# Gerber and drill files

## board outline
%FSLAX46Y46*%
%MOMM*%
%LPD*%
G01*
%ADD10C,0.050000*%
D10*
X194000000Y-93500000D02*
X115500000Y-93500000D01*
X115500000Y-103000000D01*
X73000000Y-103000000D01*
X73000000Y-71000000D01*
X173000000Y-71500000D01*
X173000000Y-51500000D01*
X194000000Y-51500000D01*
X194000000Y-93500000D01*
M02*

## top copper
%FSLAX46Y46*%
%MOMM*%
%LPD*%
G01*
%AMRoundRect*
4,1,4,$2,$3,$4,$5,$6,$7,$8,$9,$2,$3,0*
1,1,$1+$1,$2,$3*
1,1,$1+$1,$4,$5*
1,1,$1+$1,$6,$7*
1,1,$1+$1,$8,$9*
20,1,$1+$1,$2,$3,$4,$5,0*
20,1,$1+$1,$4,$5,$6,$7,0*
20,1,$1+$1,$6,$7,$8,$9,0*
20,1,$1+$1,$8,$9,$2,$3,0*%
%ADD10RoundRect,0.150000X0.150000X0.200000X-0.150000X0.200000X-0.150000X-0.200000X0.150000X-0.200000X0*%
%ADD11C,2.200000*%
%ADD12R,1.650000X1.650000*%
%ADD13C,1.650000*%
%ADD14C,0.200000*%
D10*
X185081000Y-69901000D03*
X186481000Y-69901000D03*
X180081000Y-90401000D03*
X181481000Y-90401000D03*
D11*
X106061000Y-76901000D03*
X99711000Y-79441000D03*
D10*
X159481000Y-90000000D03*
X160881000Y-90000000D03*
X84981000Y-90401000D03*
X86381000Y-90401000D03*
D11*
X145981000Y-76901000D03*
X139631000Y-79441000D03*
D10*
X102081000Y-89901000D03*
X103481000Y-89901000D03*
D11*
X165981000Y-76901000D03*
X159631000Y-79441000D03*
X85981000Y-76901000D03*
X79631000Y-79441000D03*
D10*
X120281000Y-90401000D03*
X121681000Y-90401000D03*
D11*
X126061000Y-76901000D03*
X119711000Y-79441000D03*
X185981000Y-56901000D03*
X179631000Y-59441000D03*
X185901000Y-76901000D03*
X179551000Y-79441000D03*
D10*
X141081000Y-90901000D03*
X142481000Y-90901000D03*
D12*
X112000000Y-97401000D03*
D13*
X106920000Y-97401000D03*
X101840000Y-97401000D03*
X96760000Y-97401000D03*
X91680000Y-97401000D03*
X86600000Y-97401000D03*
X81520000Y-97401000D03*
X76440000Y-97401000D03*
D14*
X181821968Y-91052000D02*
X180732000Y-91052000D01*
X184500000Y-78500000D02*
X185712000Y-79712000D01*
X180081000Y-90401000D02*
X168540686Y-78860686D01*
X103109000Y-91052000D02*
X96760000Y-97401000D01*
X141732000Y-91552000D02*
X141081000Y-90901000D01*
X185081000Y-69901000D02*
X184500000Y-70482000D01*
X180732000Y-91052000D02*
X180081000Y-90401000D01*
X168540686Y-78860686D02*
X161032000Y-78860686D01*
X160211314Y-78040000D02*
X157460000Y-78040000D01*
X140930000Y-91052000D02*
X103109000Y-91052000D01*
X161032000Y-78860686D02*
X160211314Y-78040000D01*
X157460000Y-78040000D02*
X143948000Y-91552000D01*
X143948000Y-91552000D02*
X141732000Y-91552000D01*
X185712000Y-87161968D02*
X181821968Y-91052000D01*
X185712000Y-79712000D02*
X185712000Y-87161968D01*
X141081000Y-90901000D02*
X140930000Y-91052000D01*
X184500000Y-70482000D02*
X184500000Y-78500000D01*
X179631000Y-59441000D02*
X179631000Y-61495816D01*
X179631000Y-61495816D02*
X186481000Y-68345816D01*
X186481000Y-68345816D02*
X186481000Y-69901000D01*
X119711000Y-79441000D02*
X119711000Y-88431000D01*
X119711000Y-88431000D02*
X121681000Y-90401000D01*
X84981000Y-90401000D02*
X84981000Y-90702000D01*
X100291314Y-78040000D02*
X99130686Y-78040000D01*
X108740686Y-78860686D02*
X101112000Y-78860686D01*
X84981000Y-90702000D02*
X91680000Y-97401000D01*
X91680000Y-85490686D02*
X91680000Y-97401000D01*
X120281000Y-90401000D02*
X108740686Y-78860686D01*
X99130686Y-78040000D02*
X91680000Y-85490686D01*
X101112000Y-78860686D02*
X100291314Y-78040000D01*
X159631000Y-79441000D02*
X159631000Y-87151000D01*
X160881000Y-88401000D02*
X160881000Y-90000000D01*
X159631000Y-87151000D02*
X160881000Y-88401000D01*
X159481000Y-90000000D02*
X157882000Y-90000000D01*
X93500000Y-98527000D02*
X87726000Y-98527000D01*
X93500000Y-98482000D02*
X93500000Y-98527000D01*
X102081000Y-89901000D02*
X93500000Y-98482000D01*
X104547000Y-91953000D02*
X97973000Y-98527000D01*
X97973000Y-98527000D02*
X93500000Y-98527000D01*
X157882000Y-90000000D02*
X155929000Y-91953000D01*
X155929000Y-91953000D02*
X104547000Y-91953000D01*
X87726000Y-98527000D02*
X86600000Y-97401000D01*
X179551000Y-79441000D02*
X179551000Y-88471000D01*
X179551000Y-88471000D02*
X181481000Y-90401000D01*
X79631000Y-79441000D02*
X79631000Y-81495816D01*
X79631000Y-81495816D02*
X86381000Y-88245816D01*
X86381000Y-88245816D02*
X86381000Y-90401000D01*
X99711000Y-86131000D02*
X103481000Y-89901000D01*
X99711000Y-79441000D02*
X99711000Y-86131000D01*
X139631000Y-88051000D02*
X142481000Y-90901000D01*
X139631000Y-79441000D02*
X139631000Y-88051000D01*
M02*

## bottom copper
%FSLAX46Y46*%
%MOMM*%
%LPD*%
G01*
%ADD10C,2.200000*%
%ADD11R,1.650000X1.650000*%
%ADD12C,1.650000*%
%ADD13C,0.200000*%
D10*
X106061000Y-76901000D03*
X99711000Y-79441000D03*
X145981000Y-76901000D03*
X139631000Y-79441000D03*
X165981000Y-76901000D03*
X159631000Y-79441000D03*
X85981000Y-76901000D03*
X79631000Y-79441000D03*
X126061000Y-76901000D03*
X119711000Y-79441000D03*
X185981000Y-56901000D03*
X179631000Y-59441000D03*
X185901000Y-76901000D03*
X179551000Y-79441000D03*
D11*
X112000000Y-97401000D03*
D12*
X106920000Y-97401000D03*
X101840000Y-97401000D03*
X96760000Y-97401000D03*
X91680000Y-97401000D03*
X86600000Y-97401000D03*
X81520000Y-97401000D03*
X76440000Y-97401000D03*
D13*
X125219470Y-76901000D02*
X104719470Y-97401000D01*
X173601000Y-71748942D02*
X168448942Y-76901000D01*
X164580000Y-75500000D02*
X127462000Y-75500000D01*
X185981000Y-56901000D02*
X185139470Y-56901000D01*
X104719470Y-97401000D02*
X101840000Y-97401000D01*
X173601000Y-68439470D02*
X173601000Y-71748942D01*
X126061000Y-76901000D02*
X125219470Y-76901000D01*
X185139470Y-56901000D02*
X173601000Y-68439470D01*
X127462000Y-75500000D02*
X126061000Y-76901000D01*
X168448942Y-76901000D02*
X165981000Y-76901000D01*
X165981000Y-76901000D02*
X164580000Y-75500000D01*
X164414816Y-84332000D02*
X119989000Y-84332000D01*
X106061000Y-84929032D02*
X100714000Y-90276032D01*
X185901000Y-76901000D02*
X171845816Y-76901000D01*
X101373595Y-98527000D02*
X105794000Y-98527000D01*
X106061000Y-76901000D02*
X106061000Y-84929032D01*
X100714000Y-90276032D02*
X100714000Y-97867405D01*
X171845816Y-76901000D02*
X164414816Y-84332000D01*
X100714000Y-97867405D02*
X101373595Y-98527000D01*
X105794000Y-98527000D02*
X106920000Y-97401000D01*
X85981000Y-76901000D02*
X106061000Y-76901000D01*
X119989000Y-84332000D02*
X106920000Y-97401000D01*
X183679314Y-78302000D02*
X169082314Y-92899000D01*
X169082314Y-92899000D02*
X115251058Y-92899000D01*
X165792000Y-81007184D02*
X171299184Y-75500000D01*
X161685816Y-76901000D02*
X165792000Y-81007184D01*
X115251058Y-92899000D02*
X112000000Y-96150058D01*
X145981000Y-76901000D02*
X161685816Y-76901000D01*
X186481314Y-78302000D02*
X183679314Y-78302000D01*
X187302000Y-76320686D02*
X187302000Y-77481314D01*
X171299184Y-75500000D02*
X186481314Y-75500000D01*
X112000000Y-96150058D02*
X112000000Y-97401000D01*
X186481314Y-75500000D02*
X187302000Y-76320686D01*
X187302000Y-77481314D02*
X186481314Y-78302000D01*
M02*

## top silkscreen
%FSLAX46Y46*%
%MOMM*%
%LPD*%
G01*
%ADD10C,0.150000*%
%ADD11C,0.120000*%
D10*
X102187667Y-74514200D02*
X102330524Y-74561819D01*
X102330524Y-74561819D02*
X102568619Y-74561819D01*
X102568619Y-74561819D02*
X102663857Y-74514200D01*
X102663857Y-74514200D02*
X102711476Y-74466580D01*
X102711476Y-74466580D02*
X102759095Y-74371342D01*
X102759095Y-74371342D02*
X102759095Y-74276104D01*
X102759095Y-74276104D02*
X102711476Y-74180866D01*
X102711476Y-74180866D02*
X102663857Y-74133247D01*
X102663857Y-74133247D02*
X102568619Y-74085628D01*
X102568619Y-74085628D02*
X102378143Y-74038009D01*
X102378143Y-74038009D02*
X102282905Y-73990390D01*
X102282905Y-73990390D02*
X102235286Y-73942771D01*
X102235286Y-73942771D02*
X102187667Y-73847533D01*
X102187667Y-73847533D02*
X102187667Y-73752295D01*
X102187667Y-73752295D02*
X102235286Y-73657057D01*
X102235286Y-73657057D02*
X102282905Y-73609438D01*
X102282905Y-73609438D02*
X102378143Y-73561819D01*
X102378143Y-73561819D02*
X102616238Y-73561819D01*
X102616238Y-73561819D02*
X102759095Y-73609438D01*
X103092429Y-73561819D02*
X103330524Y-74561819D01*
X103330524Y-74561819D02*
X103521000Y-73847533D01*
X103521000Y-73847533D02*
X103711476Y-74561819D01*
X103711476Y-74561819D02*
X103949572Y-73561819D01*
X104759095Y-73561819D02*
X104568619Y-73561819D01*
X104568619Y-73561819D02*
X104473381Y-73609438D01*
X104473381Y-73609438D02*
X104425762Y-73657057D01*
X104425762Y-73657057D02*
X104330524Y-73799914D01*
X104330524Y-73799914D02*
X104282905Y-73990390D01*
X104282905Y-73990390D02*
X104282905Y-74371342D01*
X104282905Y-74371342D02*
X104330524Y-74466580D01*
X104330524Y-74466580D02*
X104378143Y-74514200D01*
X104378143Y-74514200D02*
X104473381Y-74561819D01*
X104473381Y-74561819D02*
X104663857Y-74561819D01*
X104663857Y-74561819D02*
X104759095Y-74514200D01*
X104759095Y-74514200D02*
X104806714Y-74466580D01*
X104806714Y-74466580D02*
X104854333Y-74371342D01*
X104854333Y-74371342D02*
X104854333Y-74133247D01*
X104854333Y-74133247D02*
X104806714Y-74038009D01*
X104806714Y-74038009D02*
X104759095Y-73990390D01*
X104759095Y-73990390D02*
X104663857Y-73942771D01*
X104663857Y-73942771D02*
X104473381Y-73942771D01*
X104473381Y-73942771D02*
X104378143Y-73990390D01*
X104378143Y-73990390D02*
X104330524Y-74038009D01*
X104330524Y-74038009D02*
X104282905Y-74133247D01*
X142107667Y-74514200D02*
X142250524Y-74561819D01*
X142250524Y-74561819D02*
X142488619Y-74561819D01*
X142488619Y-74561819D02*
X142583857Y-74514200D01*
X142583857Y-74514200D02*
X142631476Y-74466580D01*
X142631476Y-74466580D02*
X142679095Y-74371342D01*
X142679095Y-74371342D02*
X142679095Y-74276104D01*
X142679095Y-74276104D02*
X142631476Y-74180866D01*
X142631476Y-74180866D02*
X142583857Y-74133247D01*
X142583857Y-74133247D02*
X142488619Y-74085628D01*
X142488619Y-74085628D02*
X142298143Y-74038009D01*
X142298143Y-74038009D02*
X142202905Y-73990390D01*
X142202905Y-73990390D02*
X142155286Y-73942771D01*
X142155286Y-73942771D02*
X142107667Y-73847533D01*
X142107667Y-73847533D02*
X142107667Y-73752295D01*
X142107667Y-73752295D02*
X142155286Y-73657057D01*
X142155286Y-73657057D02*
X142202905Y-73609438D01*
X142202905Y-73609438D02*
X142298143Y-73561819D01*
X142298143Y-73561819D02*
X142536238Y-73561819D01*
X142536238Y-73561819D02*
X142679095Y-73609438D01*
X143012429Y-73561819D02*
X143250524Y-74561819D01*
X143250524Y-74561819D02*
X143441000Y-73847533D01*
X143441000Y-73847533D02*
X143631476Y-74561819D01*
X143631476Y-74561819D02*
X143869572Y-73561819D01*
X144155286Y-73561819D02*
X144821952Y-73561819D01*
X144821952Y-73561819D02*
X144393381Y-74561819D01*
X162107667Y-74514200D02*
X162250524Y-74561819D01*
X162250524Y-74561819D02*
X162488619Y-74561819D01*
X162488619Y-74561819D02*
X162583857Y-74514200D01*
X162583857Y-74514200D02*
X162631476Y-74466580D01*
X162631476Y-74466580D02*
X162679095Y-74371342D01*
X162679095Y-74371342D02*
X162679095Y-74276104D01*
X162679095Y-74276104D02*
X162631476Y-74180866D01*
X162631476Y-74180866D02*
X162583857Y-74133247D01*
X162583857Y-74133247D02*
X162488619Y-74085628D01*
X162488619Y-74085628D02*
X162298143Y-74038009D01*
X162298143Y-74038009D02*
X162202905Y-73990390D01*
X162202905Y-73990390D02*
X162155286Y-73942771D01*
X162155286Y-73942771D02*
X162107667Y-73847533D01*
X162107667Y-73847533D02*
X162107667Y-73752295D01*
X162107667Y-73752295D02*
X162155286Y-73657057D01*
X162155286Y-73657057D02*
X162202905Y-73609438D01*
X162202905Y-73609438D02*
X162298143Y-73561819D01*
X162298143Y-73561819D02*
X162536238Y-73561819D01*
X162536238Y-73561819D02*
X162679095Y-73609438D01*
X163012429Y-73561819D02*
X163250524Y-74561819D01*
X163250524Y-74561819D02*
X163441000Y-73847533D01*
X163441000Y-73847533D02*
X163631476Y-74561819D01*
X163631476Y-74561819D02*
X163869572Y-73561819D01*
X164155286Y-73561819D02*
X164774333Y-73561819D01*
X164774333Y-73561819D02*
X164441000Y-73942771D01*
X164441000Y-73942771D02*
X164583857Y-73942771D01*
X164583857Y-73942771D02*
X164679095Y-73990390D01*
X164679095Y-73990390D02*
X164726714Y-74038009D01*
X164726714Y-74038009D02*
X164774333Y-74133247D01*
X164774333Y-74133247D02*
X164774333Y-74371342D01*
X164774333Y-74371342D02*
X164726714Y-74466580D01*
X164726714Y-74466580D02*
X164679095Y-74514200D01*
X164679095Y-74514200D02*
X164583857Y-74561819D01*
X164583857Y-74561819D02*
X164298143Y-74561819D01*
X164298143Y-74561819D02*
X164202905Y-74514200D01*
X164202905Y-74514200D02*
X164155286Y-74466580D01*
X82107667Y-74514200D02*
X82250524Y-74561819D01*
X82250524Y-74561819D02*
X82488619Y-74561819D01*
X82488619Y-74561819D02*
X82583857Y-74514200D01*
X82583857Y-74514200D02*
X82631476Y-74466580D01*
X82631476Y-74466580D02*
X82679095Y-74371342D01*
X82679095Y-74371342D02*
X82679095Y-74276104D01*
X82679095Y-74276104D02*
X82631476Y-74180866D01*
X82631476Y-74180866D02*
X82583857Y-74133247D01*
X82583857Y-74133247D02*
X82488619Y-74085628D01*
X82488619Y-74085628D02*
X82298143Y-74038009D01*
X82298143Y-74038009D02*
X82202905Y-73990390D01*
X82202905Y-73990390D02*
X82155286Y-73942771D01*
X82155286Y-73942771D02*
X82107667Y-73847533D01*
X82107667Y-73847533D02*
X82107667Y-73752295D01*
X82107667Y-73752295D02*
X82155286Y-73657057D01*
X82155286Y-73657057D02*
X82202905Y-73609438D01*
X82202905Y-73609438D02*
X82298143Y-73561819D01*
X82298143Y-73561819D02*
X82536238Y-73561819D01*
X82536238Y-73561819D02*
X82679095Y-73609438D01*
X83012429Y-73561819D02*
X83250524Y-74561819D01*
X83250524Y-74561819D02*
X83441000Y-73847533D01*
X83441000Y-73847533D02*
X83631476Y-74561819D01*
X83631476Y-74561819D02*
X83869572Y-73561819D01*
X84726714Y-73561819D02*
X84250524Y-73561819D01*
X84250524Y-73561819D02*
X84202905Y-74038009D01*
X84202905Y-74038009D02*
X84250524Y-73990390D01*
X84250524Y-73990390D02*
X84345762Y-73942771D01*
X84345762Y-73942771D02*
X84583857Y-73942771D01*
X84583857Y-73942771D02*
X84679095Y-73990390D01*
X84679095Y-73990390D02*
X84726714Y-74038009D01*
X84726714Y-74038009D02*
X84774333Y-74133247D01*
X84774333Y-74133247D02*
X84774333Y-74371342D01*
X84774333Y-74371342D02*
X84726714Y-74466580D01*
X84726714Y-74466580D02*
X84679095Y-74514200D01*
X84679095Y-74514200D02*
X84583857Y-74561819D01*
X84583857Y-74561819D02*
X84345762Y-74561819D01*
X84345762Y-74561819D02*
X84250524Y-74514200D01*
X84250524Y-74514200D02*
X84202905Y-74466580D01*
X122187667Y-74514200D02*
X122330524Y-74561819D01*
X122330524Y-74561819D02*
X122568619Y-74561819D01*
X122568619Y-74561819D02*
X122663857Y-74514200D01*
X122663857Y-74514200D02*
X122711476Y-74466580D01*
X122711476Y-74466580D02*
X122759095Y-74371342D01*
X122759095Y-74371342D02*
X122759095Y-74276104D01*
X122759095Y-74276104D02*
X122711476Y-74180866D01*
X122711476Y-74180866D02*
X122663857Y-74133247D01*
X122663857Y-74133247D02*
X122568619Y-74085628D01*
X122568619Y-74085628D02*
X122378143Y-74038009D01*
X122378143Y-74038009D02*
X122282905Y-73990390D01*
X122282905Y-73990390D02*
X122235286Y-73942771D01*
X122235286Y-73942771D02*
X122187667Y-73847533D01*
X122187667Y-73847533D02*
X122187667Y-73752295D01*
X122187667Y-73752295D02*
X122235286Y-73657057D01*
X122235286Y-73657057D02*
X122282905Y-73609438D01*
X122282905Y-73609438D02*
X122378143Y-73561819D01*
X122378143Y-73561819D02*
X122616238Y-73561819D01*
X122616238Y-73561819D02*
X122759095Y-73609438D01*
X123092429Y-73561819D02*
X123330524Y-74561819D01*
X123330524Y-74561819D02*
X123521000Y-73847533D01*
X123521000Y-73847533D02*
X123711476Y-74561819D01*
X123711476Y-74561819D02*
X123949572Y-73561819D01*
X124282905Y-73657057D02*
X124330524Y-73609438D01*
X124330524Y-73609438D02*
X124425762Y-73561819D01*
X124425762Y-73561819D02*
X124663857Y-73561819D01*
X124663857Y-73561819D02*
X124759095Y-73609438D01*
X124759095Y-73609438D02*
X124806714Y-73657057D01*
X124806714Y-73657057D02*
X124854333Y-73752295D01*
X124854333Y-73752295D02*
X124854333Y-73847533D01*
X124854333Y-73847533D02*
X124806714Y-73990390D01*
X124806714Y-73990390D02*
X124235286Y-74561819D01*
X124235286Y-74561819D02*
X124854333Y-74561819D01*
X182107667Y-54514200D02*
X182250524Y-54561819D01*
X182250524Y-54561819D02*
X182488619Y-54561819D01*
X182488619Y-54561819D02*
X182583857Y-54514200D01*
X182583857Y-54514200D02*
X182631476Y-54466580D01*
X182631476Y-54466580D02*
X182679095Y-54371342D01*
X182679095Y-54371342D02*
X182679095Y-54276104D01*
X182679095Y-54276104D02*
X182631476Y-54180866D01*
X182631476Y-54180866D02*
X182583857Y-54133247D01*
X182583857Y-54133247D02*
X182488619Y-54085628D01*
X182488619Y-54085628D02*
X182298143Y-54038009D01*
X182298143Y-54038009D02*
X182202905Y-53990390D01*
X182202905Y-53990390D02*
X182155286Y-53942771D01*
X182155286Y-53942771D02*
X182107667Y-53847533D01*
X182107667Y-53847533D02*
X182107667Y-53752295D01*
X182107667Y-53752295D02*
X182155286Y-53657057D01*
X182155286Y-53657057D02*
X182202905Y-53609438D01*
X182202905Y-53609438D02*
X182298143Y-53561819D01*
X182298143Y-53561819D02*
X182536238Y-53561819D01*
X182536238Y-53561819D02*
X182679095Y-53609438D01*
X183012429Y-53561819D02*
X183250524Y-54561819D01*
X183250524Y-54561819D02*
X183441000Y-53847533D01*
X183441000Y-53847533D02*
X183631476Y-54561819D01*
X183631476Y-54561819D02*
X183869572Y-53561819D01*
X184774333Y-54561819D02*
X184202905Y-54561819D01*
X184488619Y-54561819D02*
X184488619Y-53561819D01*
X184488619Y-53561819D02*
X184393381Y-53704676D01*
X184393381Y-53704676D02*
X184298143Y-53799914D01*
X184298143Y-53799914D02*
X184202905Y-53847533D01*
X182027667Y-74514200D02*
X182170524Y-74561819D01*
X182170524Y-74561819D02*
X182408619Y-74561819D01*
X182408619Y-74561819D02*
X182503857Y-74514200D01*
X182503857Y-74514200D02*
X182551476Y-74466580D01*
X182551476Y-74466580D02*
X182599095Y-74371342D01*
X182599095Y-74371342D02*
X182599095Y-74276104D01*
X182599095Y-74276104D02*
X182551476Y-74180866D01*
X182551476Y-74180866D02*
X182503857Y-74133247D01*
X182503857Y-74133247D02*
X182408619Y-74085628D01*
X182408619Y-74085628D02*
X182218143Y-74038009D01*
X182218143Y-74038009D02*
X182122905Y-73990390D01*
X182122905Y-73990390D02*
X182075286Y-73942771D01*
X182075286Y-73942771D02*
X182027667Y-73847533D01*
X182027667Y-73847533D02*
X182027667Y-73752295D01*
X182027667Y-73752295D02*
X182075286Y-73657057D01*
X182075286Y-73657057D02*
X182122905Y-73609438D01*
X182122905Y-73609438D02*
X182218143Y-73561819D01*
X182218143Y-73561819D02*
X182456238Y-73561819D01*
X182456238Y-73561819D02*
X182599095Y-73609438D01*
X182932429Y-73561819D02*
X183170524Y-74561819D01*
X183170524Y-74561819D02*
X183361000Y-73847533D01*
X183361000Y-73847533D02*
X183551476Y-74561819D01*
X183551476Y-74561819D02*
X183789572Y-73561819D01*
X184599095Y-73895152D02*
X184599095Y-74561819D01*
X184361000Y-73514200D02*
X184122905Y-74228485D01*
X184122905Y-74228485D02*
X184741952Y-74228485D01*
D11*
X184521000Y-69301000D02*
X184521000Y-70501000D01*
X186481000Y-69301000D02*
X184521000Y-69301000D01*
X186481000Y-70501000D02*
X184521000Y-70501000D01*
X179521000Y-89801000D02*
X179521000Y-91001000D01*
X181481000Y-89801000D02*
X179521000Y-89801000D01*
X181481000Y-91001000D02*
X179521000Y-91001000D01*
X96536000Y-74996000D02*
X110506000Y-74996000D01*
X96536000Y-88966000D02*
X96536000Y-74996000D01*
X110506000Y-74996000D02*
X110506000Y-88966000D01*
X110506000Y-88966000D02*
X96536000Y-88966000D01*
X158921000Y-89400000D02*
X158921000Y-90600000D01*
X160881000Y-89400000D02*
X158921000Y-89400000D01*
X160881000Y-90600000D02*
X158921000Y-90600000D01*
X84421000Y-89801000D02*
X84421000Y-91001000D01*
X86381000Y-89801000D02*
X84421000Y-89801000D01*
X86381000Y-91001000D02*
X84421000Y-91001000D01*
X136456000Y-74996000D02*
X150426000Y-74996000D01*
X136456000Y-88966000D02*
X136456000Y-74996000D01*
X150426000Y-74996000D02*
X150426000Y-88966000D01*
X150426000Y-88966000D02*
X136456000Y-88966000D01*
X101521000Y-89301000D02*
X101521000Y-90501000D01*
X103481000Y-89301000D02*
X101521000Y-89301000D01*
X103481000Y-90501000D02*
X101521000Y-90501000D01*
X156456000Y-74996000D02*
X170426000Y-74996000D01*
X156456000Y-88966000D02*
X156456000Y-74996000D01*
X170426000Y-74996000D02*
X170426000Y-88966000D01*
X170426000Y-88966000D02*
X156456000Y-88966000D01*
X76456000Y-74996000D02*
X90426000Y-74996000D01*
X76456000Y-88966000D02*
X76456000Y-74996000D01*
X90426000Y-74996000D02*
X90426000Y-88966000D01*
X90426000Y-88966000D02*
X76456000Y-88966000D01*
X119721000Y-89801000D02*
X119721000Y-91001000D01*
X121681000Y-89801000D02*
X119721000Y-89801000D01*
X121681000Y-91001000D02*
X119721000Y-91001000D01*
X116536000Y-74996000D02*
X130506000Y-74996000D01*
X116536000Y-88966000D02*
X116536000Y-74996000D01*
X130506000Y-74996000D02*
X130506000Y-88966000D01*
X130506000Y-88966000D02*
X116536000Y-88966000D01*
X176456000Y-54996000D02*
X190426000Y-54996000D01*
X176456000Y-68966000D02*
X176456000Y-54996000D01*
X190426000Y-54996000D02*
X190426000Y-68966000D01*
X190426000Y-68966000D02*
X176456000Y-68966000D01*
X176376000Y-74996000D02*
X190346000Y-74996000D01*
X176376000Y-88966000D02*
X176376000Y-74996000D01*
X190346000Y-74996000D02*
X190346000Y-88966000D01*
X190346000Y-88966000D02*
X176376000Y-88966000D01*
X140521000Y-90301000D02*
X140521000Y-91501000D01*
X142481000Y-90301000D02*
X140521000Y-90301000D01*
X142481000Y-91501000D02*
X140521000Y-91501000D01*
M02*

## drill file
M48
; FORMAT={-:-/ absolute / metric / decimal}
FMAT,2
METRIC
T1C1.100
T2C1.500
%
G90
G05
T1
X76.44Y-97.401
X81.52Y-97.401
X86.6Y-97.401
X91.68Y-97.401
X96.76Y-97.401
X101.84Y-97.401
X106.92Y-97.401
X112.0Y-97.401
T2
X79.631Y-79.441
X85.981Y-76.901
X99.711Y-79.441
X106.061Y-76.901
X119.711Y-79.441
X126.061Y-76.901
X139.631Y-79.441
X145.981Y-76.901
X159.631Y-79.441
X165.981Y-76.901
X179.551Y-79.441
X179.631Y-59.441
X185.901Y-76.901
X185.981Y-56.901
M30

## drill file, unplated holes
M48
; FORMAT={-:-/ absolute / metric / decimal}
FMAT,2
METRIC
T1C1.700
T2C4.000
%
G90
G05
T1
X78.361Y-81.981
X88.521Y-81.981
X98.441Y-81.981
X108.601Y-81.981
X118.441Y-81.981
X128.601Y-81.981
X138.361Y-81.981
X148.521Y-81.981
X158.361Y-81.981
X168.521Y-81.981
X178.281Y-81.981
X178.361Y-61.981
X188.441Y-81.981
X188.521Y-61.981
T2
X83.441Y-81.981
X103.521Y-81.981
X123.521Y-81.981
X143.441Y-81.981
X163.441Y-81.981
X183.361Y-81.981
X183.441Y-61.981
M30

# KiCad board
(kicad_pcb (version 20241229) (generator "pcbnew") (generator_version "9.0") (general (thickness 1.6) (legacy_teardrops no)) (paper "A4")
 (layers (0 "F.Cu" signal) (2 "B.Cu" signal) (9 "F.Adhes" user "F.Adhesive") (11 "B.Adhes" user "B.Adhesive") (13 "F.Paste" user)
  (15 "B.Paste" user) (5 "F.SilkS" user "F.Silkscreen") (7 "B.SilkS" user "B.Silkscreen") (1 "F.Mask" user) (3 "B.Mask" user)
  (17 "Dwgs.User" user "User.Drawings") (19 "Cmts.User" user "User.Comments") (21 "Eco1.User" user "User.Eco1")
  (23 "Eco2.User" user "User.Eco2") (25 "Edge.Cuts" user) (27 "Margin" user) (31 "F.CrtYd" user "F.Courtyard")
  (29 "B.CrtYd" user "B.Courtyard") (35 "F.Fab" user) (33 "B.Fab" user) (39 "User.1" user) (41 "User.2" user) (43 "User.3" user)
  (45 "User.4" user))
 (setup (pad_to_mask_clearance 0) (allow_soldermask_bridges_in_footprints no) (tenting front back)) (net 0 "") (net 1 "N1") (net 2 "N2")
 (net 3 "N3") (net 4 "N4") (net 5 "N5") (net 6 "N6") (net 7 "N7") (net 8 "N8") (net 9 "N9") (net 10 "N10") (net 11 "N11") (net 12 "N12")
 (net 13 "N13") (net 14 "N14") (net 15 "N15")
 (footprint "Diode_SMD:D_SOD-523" (layer "F.Cu") (at 185.781 69.901)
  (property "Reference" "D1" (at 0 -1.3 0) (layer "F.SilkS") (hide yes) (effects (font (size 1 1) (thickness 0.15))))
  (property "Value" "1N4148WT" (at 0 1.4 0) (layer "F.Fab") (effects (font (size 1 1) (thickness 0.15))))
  (fp_line (start -1.26 -0.6) (end -1.26 0.6) (stroke (width 0.12) (type solid)) (layer "F.SilkS"))
  (fp_line (start 0.7 -0.6) (end -1.26 -0.6) (stroke (width 0.12) (type solid)) (layer "F.SilkS"))
  (fp_line (start 0.7 0.6) (end -1.26 0.6) (stroke (width 0.12) (type solid)) (layer "F.SilkS"))
  (pad "1" smd roundrect (at -0.7 0 180) (size 0.6 0.7) (layers "F.Cu" "F.Mask" "F.Paste") (roundrect_rratio 0.25) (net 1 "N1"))
  (pad "2" smd roundrect (at 0.7 0 180) (size 0.6 0.7) (layers "F.Cu" "F.Mask" "F.Paste") (roundrect_rratio 0.25) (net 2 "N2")))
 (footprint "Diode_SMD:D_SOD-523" (layer "F.Cu") (at 180.781 90.401)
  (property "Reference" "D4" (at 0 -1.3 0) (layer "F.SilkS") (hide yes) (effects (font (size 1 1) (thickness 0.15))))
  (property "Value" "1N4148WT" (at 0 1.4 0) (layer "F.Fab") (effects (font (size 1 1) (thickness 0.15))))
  (fp_line (start -1.26 -0.6) (end -1.26 0.6) (stroke (width 0.12) (type solid)) (layer "F.SilkS"))
  (fp_line (start 0.7 -0.6) (end -1.26 -0.6) (stroke (width 0.12) (type solid)) (layer "F.SilkS"))
  (fp_line (start 0.7 0.6) (end -1.26 0.6) (stroke (width 0.12) (type solid)) (layer "F.SilkS"))
  (pad "1" smd roundrect (at -0.7 0 180) (size 0.6 0.7) (layers "F.Cu" "F.Mask" "F.Paste") (roundrect_rratio 0.25) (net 1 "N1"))
  (pad "2" smd roundrect (at 0.7 0 180) (size 0.6 0.7) (layers "F.Cu" "F.Mask" "F.Paste") (roundrect_rratio 0.25) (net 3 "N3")))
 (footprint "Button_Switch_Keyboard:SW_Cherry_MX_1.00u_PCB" (layer "F.Cu") (at 106.061 76.901)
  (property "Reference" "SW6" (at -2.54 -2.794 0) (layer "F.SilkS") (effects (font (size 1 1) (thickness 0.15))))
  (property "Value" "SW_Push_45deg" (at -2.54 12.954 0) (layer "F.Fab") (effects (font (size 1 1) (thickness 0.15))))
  (fp_line (start -9.525 -1.905) (end 4.445 -1.905) (stroke (width 0.12) (type solid)) (layer "F.SilkS"))
  (fp_line (start -9.525 12.065) (end -9.525 -1.905) (stroke (width 0.12) (type solid)) (layer "F.SilkS"))
  (fp_line (start 4.445 -1.905) (end 4.445 12.065) (stroke (width 0.12) (type solid)) (layer "F.SilkS"))
  (fp_line (start 4.445 12.065) (end -9.525 12.065) (stroke (width 0.12) (type solid)) (layer "F.SilkS"))
  (pad "" np_thru_hole circle (at -7.62 5.08) (size 1.7 1.7) (drill 1.7) (layers "*.Cu" "*.Mask"))
  (pad "" np_thru_hole circle (at -2.54 5.08) (size 4 4) (drill 4) (layers "*.Cu" "*.Mask"))
  (pad "" np_thru_hole circle (at 2.54 5.08) (size 1.7 1.7) (drill 1.7) (layers "*.Cu" "*.Mask"))
  (pad "1" thru_hole circle (at 0 0) (size 2.2 2.2) (drill 1.5) (layers "*.Cu" "*.Mask") (remove_unused_layers no) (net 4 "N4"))
  (pad "2" thru_hole circle (at -6.35 2.54) (size 2.2 2.2) (drill 1.5) (layers "*.Cu" "*.Mask") (remove_unused_layers no) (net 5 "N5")))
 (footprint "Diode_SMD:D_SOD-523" (layer "F.Cu") (at 160.181 90)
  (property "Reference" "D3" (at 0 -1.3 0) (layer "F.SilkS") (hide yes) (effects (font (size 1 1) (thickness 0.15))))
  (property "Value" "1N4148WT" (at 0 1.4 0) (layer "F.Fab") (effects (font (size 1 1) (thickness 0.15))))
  (fp_line (start -1.26 -0.6) (end -1.26 0.6) (stroke (width 0.12) (type solid)) (layer "F.SilkS"))
  (fp_line (start 0.7 -0.6) (end -1.26 -0.6) (stroke (width 0.12) (type solid)) (layer "F.SilkS"))
  (fp_line (start 0.7 0.6) (end -1.26 0.6) (stroke (width 0.12) (type solid)) (layer "F.SilkS"))
  (pad "1" smd roundrect (at -0.7 0 180) (size 0.6 0.7) (layers "F.Cu" "F.Mask" "F.Paste") (roundrect_rratio 0.25) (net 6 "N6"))
  (pad "2" smd roundrect (at 0.7 0 180) (size 0.6 0.7) (layers "F.Cu" "F.Mask" "F.Paste") (roundrect_rratio 0.25) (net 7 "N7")))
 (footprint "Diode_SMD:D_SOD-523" (layer "F.Cu") (at 85.681 90.401)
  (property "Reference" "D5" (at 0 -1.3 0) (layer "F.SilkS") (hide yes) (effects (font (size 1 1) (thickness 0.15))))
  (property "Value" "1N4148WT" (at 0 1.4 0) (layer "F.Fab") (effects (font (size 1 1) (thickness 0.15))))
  (fp_line (start -1.26 -0.6) (end -1.26 0.6) (stroke (width 0.12) (type solid)) (layer "F.SilkS"))
  (fp_line (start 0.7 -0.6) (end -1.26 -0.6) (stroke (width 0.12) (type solid)) (layer "F.SilkS"))
  (fp_line (start 0.7 0.6) (end -1.26 0.6) (stroke (width 0.12) (type solid)) (layer "F.SilkS"))
  (pad "1" smd roundrect (at -0.7 0 180) (size 0.6 0.7) (layers "F.Cu" "F.Mask" "F.Paste") (roundrect_rratio 0.25) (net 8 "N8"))
  (pad "2" smd roundrect (at 0.7 0 180) (size 0.6 0.7) (layers "F.Cu" "F.Mask" "F.Paste") (roundrect_rratio 0.25) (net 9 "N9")))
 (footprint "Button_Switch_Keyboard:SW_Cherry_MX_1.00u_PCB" (layer "F.Cu") (at 145.981 76.901)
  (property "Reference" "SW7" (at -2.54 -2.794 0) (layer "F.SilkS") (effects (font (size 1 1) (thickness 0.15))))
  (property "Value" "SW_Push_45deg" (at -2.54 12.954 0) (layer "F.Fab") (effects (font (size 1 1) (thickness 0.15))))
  (fp_line (start -9.525 -1.905) (end 4.445 -1.905) (stroke (width 0.12) (type solid)) (layer "F.SilkS"))
  (fp_line (start -9.525 12.065) (end -9.525 -1.905) (stroke (width 0.12) (type solid)) (layer "F.SilkS"))
  (fp_line (start 4.445 -1.905) (end 4.445 12.065) (stroke (width 0.12) (type solid)) (layer "F.SilkS"))
  (fp_line (start 4.445 12.065) (end -9.525 12.065) (stroke (width 0.12) (type solid)) (layer "F.SilkS"))
  (pad "" np_thru_hole circle (at -7.62 5.08) (size 1.7 1.7) (drill 1.7) (layers "*.Cu" "*.Mask"))
  (pad "" np_thru_hole circle (at -2.54 5.08) (size 4 4) (drill 4) (layers "*.Cu" "*.Mask"))
  (pad "" np_thru_hole circle (at 2.54 5.08) (size 1.7 1.7) (drill 1.7) (layers "*.Cu" "*.Mask"))
  (pad "1" thru_hole circle (at 0 0) (size 2.2 2.2) (drill 1.5) (layers "*.Cu" "*.Mask") (remove_unused_layers no) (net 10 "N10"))
  (pad "2" thru_hole circle (at -6.35 2.54) (size 2.2 2.2) (drill 1.5) (layers "*.Cu" "*.Mask") (remove_unused_layers no) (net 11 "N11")))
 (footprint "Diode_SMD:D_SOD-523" (layer "F.Cu") (at 102.781 89.901)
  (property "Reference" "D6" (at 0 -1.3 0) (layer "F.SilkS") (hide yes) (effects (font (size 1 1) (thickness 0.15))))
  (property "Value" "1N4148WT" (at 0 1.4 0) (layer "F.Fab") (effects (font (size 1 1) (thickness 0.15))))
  (fp_line (start -1.26 -0.6) (end -1.26 0.6) (stroke (width 0.12) (type solid)) (layer "F.SilkS"))
  (fp_line (start 0.7 -0.6) (end -1.26 -0.6) (stroke (width 0.12) (type solid)) (layer "F.SilkS"))
  (fp_line (start 0.7 0.6) (end -1.26 0.6) (stroke (width 0.12) (type solid)) (layer "F.SilkS"))
  (pad "1" smd roundrect (at -0.7 0 180) (size 0.6 0.7) (layers "F.Cu" "F.Mask" "F.Paste") (roundrect_rratio 0.25) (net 6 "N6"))
  (pad "2" smd roundrect (at 0.7 0 180) (size 0.6 0.7) (layers "F.Cu" "F.Mask" "F.Paste") (roundrect_rratio 0.25) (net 5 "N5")))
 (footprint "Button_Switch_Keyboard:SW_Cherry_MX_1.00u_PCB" (layer "F.Cu") (at 165.981 76.901)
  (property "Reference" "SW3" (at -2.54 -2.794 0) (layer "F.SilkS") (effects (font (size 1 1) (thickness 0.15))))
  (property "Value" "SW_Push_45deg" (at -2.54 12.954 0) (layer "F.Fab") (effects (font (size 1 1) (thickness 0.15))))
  (fp_line (start -9.525 -1.905) (end 4.445 -1.905) (stroke (width 0.12) (type solid)) (layer "F.SilkS"))
  (fp_line (start -9.525 12.065) (end -9.525 -1.905) (stroke (width 0.12) (type solid)) (layer "F.SilkS"))
  (fp_line (start 4.445 -1.905) (end 4.445 12.065) (stroke (width 0.12) (type solid)) (layer "F.SilkS"))
  (fp_line (start 4.445 12.065) (end -9.525 12.065) (stroke (width 0.12) (type solid)) (layer "F.SilkS"))
  (pad "" np_thru_hole circle (at -7.62 5.08) (size 1.7 1.7) (drill 1.7) (layers "*.Cu" "*.Mask"))
  (pad "" np_thru_hole circle (at -2.54 5.08) (size 4 4) (drill 4) (layers "*.Cu" "*.Mask"))
  (pad "" np_thru_hole circle (at 2.54 5.08) (size 1.7 1.7) (drill 1.7) (layers "*.Cu" "*.Mask"))
  (pad "1" thru_hole circle (at 0 0) (size 2.2 2.2) (drill 1.5) (layers "*.Cu" "*.Mask") (remove_unused_layers no) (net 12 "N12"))
  (pad "2" thru_hole circle (at -6.35 2.54) (size 2.2 2.2) (drill 1.5) (layers "*.Cu" "*.Mask") (remove_unused_layers no) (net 7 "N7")))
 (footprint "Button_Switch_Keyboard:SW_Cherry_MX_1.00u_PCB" (layer "F.Cu") (at 85.981 76.901)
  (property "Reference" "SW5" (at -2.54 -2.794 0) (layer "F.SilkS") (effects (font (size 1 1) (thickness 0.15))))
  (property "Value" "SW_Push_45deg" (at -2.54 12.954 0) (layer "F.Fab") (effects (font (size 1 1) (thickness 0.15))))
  (fp_line (start -9.525 -1.905) (end 4.445 -1.905) (stroke (width 0.12) (type solid)) (layer "F.SilkS"))
  (fp_line (start -9.525 12.065) (end -9.525 -1.905) (stroke (width 0.12) (type solid)) (layer "F.SilkS"))
  (fp_line (start 4.445 -1.905) (end 4.445 12.065) (stroke (width 0.12) (type solid)) (layer "F.SilkS"))
  (fp_line (start 4.445 12.065) (end -9.525 12.065) (stroke (width 0.12) (type solid)) (layer "F.SilkS"))
  (pad "" np_thru_hole circle (at -7.62 5.08) (size 1.7 1.7) (drill 1.7) (layers "*.Cu" "*.Mask"))
  (pad "" np_thru_hole circle (at -2.54 5.08) (size 4 4) (drill 4) (layers "*.Cu" "*.Mask"))
  (pad "" np_thru_hole circle (at 2.54 5.08) (size 1.7 1.7) (drill 1.7) (layers "*.Cu" "*.Mask"))
  (pad "1" thru_hole circle (at 0 0) (size 2.2 2.2) (drill 1.5) (layers "*.Cu" "*.Mask") (remove_unused_layers no) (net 4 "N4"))
  (pad "2" thru_hole circle (at -6.35 2.54) (size 2.2 2.2) (drill 1.5) (layers "*.Cu" "*.Mask") (remove_unused_layers no) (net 9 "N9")))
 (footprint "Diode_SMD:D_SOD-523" (layer "F.Cu") (at 120.981 90.401)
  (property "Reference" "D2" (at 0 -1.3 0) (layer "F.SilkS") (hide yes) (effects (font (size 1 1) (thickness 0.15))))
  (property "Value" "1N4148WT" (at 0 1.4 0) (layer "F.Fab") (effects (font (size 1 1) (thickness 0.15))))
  (fp_line (start -1.26 -0.6) (end -1.26 0.6) (stroke (width 0.12) (type solid)) (layer "F.SilkS"))
  (fp_line (start 0.7 -0.6) (end -1.26 -0.6) (stroke (width 0.12) (type solid)) (layer "F.SilkS"))
  (fp_line (start 0.7 0.6) (end -1.26 0.6) (stroke (width 0.12) (type solid)) (layer "F.SilkS"))
  (pad "1" smd roundrect (at -0.7 0 180) (size 0.6 0.7) (layers "F.Cu" "F.Mask" "F.Paste") (roundrect_rratio 0.25) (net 8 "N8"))
  (pad "2" smd roundrect (at 0.7 0 180) (size 0.6 0.7) (layers "F.Cu" "F.Mask" "F.Paste") (roundrect_rratio 0.25) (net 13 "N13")))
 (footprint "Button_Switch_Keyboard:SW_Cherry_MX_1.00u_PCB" (layer "F.Cu") (at 126.061 76.901)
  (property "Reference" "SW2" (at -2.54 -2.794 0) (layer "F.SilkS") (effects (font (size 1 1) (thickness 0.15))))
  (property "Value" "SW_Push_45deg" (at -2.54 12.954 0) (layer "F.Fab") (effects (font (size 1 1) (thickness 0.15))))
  (fp_line (start -9.525 -1.905) (end 4.445 -1.905) (stroke (width 0.12) (type solid)) (layer "F.SilkS"))
  (fp_line (start -9.525 12.065) (end -9.525 -1.905) (stroke (width 0.12) (type solid)) (layer "F.SilkS"))
  (fp_line (start 4.445 -1.905) (end 4.445 12.065) (stroke (width 0.12) (type solid)) (layer "F.SilkS"))
  (fp_line (start 4.445 12.065) (end -9.525 12.065) (stroke (width 0.12) (type solid)) (layer "F.SilkS"))
  (pad "" np_thru_hole circle (at -7.62 5.08) (size 1.7 1.7) (drill 1.7) (layers "*.Cu" "*.Mask"))
  (pad "" np_thru_hole circle (at -2.54 5.08) (size 4 4) (drill 4) (layers "*.Cu" "*.Mask"))
  (pad "" np_thru_hole circle (at 2.54 5.08) (size 1.7 1.7) (drill 1.7) (layers "*.Cu" "*.Mask"))
  (pad "1" thru_hole circle (at 0 0) (size 2.2 2.2) (drill 1.5) (layers "*.Cu" "*.Mask") (remove_unused_layers no) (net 12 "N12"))
  (pad "2" thru_hole circle (at -6.35 2.54) (size 2.2 2.2) (drill 1.5) (layers "*.Cu" "*.Mask") (remove_unused_layers no) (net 13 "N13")))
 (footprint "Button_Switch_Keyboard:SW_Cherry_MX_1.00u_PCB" (layer "F.Cu") (at 185.981 56.901)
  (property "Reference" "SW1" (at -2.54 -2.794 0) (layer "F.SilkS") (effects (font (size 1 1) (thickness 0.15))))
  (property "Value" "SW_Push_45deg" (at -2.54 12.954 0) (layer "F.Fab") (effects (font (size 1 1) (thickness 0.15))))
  (fp_line (start -9.525 -1.905) (end 4.445 -1.905) (stroke (width 0.12) (type solid)) (layer "F.SilkS"))
  (fp_line (start -9.525 12.065) (end -9.525 -1.905) (stroke (width 0.12) (type solid)) (layer "F.SilkS"))
  (fp_line (start 4.445 -1.905) (end 4.445 12.065) (stroke (width 0.12) (type solid)) (layer "F.SilkS"))
  (fp_line (start 4.445 12.065) (end -9.525 12.065) (stroke (width 0.12) (type solid)) (layer "F.SilkS"))
  (pad "" np_thru_hole circle (at -7.62 5.08) (size 1.7 1.7) (drill 1.7) (layers "*.Cu" "*.Mask"))
  (pad "" np_thru_hole circle (at -2.54 5.08) (size 4 4) (drill 4) (layers "*.Cu" "*.Mask"))
  (pad "" np_thru_hole circle (at 2.54 5.08) (size 1.7 1.7) (drill 1.7) (layers "*.Cu" "*.Mask"))
  (pad "1" thru_hole circle (at 0 0) (size 2.2 2.2) (drill 1.5) (layers "*.Cu" "*.Mask") (remove_unused_layers no) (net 12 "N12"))
  (pad "2" thru_hole circle (at -6.35 2.54) (size 2.2 2.2) (drill 1.5) (layers "*.Cu" "*.Mask") (remove_unused_layers no) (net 2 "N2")))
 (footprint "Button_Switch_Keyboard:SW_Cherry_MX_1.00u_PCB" (layer "F.Cu") (at 185.901 76.901)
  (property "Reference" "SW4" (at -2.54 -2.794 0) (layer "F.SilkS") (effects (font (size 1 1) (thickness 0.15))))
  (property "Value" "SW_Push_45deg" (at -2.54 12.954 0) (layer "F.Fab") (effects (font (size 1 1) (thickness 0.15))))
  (fp_line (start -9.525 -1.905) (end 4.445 -1.905) (stroke (width 0.12) (type solid)) (layer "F.SilkS"))
  (fp_line (start -9.525 12.065) (end -9.525 -1.905) (stroke (width 0.12) (type solid)) (layer "F.SilkS"))
  (fp_line (start 4.445 -1.905) (end 4.445 12.065) (stroke (width 0.12) (type solid)) (layer "F.SilkS"))
  (fp_line (start 4.445 12.065) (end -9.525 12.065) (stroke (width 0.12) (type solid)) (layer "F.SilkS"))
  (pad "" np_thru_hole circle (at -7.62 5.08) (size 1.7 1.7) (drill 1.7) (layers "*.Cu" "*.Mask"))
  (pad "" np_thru_hole circle (at -2.54 5.08) (size 4 4) (drill 4) (layers "*.Cu" "*.Mask"))
  (pad "" np_thru_hole circle (at 2.54 5.08) (size 1.7 1.7) (drill 1.7) (layers "*.Cu" "*.Mask"))
  (pad "1" thru_hole circle (at 0 0) (size 2.2 2.2) (drill 1.5) (layers "*.Cu" "*.Mask") (remove_unused_layers no) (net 4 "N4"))
  (pad "2" thru_hole circle (at -6.35 2.54) (size 2.2 2.2) (drill 1.5) (layers "*.Cu" "*.Mask") (remove_unused_layers no) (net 3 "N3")))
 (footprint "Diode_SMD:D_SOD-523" (layer "F.Cu") (at 141.781 90.901)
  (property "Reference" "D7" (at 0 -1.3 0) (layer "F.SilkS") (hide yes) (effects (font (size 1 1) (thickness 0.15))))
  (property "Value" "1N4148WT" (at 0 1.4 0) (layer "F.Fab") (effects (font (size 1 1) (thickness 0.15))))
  (fp_line (start -1.26 -0.6) (end -1.26 0.6) (stroke (width 0.12) (type solid)) (layer "F.SilkS"))
  (fp_line (start 0.7 -0.6) (end -1.26 -0.6) (stroke (width 0.12) (type solid)) (layer "F.SilkS"))
  (fp_line (start 0.7 0.6) (end -1.26 0.6) (stroke (width 0.12) (type solid)) (layer "F.SilkS"))
  (pad "1" smd roundrect (at -0.7 0 180) (size 0.6 0.7) (layers "F.Cu" "F.Mask" "F.Paste") (roundrect_rratio 0.25) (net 1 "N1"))
  (pad "2" smd roundrect (at 0.7 0 180) (size 0.6 0.7) (layers "F.Cu" "F.Mask" "F.Paste") (roundrect_rratio 0.25) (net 11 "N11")))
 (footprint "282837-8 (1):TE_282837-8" (layer "B.Cu") (at 112 97.401 180)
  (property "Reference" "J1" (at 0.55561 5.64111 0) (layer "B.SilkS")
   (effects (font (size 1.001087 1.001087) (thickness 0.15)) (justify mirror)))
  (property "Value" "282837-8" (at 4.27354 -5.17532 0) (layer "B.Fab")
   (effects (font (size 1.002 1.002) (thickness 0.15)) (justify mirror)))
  (pad "1" thru_hole rect (at 0 0 180) (size 1.65 1.65) (drill 1.1) (layers "*.Cu" "*.Mask") (remove_unused_layers no) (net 10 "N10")
   (solder_mask_margin 0.102))
  (pad "2" thru_hole circle (at 5.08 0 180) (size 1.65 1.65) (drill 1.1) (layers "*.Cu" "*.Mask") (remove_unused_layers no) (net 4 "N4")
   (solder_mask_margin 0.102))
  (pad "3" thru_hole circle (at 10.16 0 180) (size 1.65 1.65) (drill 1.1) (layers "*.Cu" "*.Mask") (remove_unused_layers no) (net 12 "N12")
   (solder_mask_margin 0.102))
  (pad "4" thru_hole circle (at 15.24 0 180) (size 1.65 1.65) (drill 1.1) (layers "*.Cu" "*.Mask") (remove_unused_layers no) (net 1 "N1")
   (solder_mask_margin 0.102))
  (pad "5" thru_hole circle (at 20.32 0 180) (size 1.65 1.65) (drill 1.1) (layers "*.Cu" "*.Mask") (remove_unused_layers no) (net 8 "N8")
   (solder_mask_margin 0.102))
  (pad "6" thru_hole circle (at 25.4 0 180) (size 1.65 1.65) (drill 1.1) (layers "*.Cu" "*.Mask") (remove_unused_layers no) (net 6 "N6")
   (solder_mask_margin 0.102))
  (pad "7" thru_hole circle (at 30.48 0 180) (size 1.65 1.65) (drill 1.1) (layers "*.Cu" "*.Mask") (remove_unused_layers no) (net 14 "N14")
   (solder_mask_margin 0.102))
  (pad "8" thru_hole circle (at 35.56 0 180) (size 1.65 1.65) (drill 1.1) (layers "*.Cu" "*.Mask") (remove_unused_layers no) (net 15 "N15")
   (solder_mask_margin 0.102)))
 (gr_poly
  (pts (xy 173 71.5) (xy 173 51.5) (xy 194 51.5) (xy 194 93.5) (xy 115.5 93.5) (xy 115.5 103) (xy 73 103) (xy 73 71))
  (stroke (width 0.05) (type solid)) (fill no) (layer "Edge.Cuts"))
 (segment (start 181.821968 91.052) (end 180.732 91.052) (width 0.2) (layer "F.Cu") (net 1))
 (segment (start 184.5 78.5) (end 185.712 79.712) (width 0.2) (layer "F.Cu") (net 1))
 (segment (start 180.081 90.401) (end 168.540686 78.860686) (width 0.2) (layer "F.Cu") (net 1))
 (segment (start 103.109 91.052) (end 96.76 97.401) (width 0.2) (layer "F.Cu") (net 1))
 (segment (start 141.732 91.552) (end 141.081 90.901) (width 0.2) (layer "F.Cu") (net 1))
 (segment (start 185.081 69.901) (end 184.5 70.482) (width 0.2) (layer "F.Cu") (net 1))
 (segment (start 180.732 91.052) (end 180.081 90.401) (width 0.2) (layer "F.Cu") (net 1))
 (segment (start 168.540686 78.860686) (end 161.032 78.860686) (width 0.2) (layer "F.Cu") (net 1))
 (segment (start 160.211314 78.04) (end 157.46 78.04) (width 0.2) (layer "F.Cu") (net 1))
 (segment (start 140.93 91.052) (end 103.109 91.052) (width 0.2) (layer "F.Cu") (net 1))
 (segment (start 161.032 78.860686) (end 160.211314 78.04) (width 0.2) (layer "F.Cu") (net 1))
 (segment (start 157.46 78.04) (end 143.948 91.552) (width 0.2) (layer "F.Cu") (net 1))
 (segment (start 143.948 91.552) (end 141.732 91.552) (width 0.2) (layer "F.Cu") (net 1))
 (segment (start 185.712 87.161968) (end 181.821968 91.052) (width 0.2) (layer "F.Cu") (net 1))
 (segment (start 185.712 79.712) (end 185.712 87.161968) (width 0.2) (layer "F.Cu") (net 1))
 (segment (start 141.081 90.901) (end 140.93 91.052) (width 0.2) (layer "F.Cu") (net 1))
 (segment (start 184.5 70.482) (end 184.5 78.5) (width 0.2) (layer "F.Cu") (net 1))
 (segment (start 179.631 59.441) (end 179.631 61.495816) (width 0.2) (layer "F.Cu") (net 2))
 (segment (start 179.631 61.495816) (end 186.481 68.345816) (width 0.2) (layer "F.Cu") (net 2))
 (segment (start 186.481 68.345816) (end 186.481 69.901) (width 0.2) (layer "F.Cu") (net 2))
 (segment (start 119.711 79.441) (end 119.711 88.431) (width 0.2) (layer "F.Cu") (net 13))
 (segment (start 119.711 88.431) (end 121.681 90.401) (width 0.2) (layer "F.Cu") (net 13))
 (segment (start 84.981 90.401) (end 84.981 90.702) (width 0.2) (layer "F.Cu") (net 8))
 (segment (start 100.291314 78.04) (end 99.130686 78.04) (width 0.2) (layer "F.Cu") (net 8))
 (segment (start 108.740686 78.860686) (end 101.112 78.860686) (width 0.2) (layer "F.Cu") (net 8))
 (segment (start 84.981 90.702) (end 91.68 97.401) (width 0.2) (layer "F.Cu") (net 8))
 (segment (start 91.68 85.490686) (end 91.68 97.401) (width 0.2) (layer "F.Cu") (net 8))
 (segment (start 120.281 90.401) (end 108.740686 78.860686) (width 0.2) (layer "F.Cu") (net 8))
 (segment (start 99.130686 78.04) (end 91.68 85.490686) (width 0.2) (layer "F.Cu") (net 8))
 (segment (start 101.112 78.860686) (end 100.291314 78.04) (width 0.2) (layer "F.Cu") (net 8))
 (segment (start 159.631 79.441) (end 159.631 87.151) (width 0.2) (layer "F.Cu") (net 7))
 (segment (start 160.881 88.401) (end 160.881 90) (width 0.2) (layer "F.Cu") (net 7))
 (segment (start 159.631 87.151) (end 160.881 88.401) (width 0.2) (layer "F.Cu") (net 7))
 (segment (start 159.481 90) (end 157.882 90) (width 0.2) (layer "F.Cu") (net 6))
 (segment (start 93.5 98.527) (end 87.726 98.527) (width 0.2) (layer "F.Cu") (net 6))
 (segment (start 93.5 98.482) (end 93.5 98.527) (width 0.2) (layer "F.Cu") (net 6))
 (segment (start 102.081 89.901) (end 93.5 98.482) (width 0.2) (layer "F.Cu") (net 6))
 (segment (start 104.547 91.953) (end 97.973 98.527) (width 0.2) (layer "F.Cu") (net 6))
 (segment (start 97.973 98.527) (end 93.5 98.527) (width 0.2) (layer "F.Cu") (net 6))
 (segment (start 157.882 90) (end 155.929 91.953) (width 0.2) (layer "F.Cu") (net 6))
 (segment (start 155.929 91.953) (end 104.547 91.953) (width 0.2) (layer "F.Cu") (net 6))
 (segment (start 87.726 98.527) (end 86.6 97.401) (width 0.2) (layer "F.Cu") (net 6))
 (segment (start 179.551 79.441) (end 179.551 88.471) (width 0.2) (layer "F.Cu") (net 3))
 (segment (start 179.551 88.471) (end 181.481 90.401) (width 0.2) (layer "F.Cu") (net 3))
 (segment (start 79.631 79.441) (end 79.631 81.495816) (width 0.2) (layer "F.Cu") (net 9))
 (segment (start 79.631 81.495816) (end 86.381 88.245816) (width 0.2) (layer "F.Cu") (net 9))
 (segment (start 86.381 88.245816) (end 86.381 90.401) (width 0.2) (layer "F.Cu") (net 9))
 (segment (start 99.711 86.131) (end 103.481 89.901) (width 0.2) (layer "F.Cu") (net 5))
 (segment (start 99.711 79.441) (end 99.711 86.131) (width 0.2) (layer "F.Cu") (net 5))
 (segment (start 139.631 88.051) (end 142.481 90.901) (width 0.2) (layer "F.Cu") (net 11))
 (segment (start 139.631 79.441) (end 139.631 88.051) (width 0.2) (layer "F.Cu") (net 11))
 (segment (start 125.21947 76.901) (end 104.71947 97.401) (width 0.2) (layer "B.Cu") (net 12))
 (segment (start 173.601 71.748942) (end 168.448942 76.901) (width 0.2) (layer "B.Cu") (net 12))
 (segment (start 164.58 75.5) (end 127.462 75.5) (width 0.2) (layer "B.Cu") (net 12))
 (segment (start 185.981 56.901) (end 185.13947 56.901) (width 0.2) (layer "B.Cu") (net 12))
 (segment (start 104.71947 97.401) (end 101.84 97.401) (width 0.2) (layer "B.Cu") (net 12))
 (segment (start 173.601 68.43947) (end 173.601 71.748942) (width 0.2) (layer "B.Cu") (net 12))
 (segment (start 126.061 76.901) (end 125.21947 76.901) (width 0.2) (layer "B.Cu") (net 12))
 (segment (start 185.13947 56.901) (end 173.601 68.43947) (width 0.2) (layer "B.Cu") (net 12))
 (segment (start 127.462 75.5) (end 126.061 76.901) (width 0.2) (layer "B.Cu") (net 12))
 (segment (start 168.448942 76.901) (end 165.981 76.901) (width 0.2) (layer "B.Cu") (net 12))
 (segment (start 165.981 76.901) (end 164.58 75.5) (width 0.2) (layer "B.Cu") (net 12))
 (segment (start 164.414816 84.332) (end 119.989 84.332) (width 0.2) (layer "B.Cu") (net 4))
 (segment (start 106.061 84.929032) (end 100.714 90.276032) (width 0.2) (layer "B.Cu") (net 4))
 (segment (start 185.901 76.901) (end 171.845816 76.901) (width 0.2) (layer "B.Cu") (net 4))
 (segment (start 101.373595 98.527) (end 105.794 98.527) (width 0.2) (layer "B.Cu") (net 4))
 (segment (start 106.061 76.901) (end 106.061 84.929032) (width 0.2) (layer "B.Cu") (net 4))
 (segment (start 100.714 90.276032) (end 100.714 97.867405) (width 0.2) (layer "B.Cu") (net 4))
 (segment (start 171.845816 76.901) (end 164.414816 84.332) (width 0.2) (layer "B.Cu") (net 4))
 (segment (start 100.714 97.867405) (end 101.373595 98.527) (width 0.2) (layer "B.Cu") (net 4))
 (segment (start 105.794 98.527) (end 106.92 97.401) (width 0.2) (layer "B.Cu") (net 4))
 (segment (start 85.981 76.901) (end 106.061 76.901) (width 0.2) (layer "B.Cu") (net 4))
 (segment (start 119.989 84.332) (end 106.92 97.401) (width 0.2) (layer "B.Cu") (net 4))
 (segment (start 183.679314 78.302) (end 169.082314 92.899) (width 0.2) (layer "B.Cu") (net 10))
 (segment (start 169.082314 92.899) (end 115.251058 92.899) (width 0.2) (layer "B.Cu") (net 10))
 (segment (start 165.792 81.007184) (end 171.299184 75.5) (width 0.2) (layer "B.Cu") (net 10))
 (segment (start 161.685816 76.901) (end 165.792 81.007184) (width 0.2) (layer "B.Cu") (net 10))
 (segment (start 115.251058 92.899) (end 112 96.150058) (width 0.2) (layer "B.Cu") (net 10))
 (segment (start 145.981 76.901) (end 161.685816 76.901) (width 0.2) (layer "B.Cu") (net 10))
 (segment (start 186.481314 78.302) (end 183.679314 78.302) (width 0.2) (layer "B.Cu") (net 10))
 (segment (start 187.302 76.320686) (end 187.302 77.481314) (width 0.2) (layer "B.Cu") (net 10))
 (segment (start 171.299184 75.5) (end 186.481314 75.5) (width 0.2) (layer "B.Cu") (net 10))
 (segment (start 112 96.150058) (end 112 97.401) (width 0.2) (layer "B.Cu") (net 10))
 (segment (start 186.481314 75.5) (end 187.302 76.320686) (width 0.2) (layer "B.Cu") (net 10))
 (segment (start 187.302 77.481314) (end 186.481314 78.302) (width 0.2) (layer "B.Cu") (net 10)))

